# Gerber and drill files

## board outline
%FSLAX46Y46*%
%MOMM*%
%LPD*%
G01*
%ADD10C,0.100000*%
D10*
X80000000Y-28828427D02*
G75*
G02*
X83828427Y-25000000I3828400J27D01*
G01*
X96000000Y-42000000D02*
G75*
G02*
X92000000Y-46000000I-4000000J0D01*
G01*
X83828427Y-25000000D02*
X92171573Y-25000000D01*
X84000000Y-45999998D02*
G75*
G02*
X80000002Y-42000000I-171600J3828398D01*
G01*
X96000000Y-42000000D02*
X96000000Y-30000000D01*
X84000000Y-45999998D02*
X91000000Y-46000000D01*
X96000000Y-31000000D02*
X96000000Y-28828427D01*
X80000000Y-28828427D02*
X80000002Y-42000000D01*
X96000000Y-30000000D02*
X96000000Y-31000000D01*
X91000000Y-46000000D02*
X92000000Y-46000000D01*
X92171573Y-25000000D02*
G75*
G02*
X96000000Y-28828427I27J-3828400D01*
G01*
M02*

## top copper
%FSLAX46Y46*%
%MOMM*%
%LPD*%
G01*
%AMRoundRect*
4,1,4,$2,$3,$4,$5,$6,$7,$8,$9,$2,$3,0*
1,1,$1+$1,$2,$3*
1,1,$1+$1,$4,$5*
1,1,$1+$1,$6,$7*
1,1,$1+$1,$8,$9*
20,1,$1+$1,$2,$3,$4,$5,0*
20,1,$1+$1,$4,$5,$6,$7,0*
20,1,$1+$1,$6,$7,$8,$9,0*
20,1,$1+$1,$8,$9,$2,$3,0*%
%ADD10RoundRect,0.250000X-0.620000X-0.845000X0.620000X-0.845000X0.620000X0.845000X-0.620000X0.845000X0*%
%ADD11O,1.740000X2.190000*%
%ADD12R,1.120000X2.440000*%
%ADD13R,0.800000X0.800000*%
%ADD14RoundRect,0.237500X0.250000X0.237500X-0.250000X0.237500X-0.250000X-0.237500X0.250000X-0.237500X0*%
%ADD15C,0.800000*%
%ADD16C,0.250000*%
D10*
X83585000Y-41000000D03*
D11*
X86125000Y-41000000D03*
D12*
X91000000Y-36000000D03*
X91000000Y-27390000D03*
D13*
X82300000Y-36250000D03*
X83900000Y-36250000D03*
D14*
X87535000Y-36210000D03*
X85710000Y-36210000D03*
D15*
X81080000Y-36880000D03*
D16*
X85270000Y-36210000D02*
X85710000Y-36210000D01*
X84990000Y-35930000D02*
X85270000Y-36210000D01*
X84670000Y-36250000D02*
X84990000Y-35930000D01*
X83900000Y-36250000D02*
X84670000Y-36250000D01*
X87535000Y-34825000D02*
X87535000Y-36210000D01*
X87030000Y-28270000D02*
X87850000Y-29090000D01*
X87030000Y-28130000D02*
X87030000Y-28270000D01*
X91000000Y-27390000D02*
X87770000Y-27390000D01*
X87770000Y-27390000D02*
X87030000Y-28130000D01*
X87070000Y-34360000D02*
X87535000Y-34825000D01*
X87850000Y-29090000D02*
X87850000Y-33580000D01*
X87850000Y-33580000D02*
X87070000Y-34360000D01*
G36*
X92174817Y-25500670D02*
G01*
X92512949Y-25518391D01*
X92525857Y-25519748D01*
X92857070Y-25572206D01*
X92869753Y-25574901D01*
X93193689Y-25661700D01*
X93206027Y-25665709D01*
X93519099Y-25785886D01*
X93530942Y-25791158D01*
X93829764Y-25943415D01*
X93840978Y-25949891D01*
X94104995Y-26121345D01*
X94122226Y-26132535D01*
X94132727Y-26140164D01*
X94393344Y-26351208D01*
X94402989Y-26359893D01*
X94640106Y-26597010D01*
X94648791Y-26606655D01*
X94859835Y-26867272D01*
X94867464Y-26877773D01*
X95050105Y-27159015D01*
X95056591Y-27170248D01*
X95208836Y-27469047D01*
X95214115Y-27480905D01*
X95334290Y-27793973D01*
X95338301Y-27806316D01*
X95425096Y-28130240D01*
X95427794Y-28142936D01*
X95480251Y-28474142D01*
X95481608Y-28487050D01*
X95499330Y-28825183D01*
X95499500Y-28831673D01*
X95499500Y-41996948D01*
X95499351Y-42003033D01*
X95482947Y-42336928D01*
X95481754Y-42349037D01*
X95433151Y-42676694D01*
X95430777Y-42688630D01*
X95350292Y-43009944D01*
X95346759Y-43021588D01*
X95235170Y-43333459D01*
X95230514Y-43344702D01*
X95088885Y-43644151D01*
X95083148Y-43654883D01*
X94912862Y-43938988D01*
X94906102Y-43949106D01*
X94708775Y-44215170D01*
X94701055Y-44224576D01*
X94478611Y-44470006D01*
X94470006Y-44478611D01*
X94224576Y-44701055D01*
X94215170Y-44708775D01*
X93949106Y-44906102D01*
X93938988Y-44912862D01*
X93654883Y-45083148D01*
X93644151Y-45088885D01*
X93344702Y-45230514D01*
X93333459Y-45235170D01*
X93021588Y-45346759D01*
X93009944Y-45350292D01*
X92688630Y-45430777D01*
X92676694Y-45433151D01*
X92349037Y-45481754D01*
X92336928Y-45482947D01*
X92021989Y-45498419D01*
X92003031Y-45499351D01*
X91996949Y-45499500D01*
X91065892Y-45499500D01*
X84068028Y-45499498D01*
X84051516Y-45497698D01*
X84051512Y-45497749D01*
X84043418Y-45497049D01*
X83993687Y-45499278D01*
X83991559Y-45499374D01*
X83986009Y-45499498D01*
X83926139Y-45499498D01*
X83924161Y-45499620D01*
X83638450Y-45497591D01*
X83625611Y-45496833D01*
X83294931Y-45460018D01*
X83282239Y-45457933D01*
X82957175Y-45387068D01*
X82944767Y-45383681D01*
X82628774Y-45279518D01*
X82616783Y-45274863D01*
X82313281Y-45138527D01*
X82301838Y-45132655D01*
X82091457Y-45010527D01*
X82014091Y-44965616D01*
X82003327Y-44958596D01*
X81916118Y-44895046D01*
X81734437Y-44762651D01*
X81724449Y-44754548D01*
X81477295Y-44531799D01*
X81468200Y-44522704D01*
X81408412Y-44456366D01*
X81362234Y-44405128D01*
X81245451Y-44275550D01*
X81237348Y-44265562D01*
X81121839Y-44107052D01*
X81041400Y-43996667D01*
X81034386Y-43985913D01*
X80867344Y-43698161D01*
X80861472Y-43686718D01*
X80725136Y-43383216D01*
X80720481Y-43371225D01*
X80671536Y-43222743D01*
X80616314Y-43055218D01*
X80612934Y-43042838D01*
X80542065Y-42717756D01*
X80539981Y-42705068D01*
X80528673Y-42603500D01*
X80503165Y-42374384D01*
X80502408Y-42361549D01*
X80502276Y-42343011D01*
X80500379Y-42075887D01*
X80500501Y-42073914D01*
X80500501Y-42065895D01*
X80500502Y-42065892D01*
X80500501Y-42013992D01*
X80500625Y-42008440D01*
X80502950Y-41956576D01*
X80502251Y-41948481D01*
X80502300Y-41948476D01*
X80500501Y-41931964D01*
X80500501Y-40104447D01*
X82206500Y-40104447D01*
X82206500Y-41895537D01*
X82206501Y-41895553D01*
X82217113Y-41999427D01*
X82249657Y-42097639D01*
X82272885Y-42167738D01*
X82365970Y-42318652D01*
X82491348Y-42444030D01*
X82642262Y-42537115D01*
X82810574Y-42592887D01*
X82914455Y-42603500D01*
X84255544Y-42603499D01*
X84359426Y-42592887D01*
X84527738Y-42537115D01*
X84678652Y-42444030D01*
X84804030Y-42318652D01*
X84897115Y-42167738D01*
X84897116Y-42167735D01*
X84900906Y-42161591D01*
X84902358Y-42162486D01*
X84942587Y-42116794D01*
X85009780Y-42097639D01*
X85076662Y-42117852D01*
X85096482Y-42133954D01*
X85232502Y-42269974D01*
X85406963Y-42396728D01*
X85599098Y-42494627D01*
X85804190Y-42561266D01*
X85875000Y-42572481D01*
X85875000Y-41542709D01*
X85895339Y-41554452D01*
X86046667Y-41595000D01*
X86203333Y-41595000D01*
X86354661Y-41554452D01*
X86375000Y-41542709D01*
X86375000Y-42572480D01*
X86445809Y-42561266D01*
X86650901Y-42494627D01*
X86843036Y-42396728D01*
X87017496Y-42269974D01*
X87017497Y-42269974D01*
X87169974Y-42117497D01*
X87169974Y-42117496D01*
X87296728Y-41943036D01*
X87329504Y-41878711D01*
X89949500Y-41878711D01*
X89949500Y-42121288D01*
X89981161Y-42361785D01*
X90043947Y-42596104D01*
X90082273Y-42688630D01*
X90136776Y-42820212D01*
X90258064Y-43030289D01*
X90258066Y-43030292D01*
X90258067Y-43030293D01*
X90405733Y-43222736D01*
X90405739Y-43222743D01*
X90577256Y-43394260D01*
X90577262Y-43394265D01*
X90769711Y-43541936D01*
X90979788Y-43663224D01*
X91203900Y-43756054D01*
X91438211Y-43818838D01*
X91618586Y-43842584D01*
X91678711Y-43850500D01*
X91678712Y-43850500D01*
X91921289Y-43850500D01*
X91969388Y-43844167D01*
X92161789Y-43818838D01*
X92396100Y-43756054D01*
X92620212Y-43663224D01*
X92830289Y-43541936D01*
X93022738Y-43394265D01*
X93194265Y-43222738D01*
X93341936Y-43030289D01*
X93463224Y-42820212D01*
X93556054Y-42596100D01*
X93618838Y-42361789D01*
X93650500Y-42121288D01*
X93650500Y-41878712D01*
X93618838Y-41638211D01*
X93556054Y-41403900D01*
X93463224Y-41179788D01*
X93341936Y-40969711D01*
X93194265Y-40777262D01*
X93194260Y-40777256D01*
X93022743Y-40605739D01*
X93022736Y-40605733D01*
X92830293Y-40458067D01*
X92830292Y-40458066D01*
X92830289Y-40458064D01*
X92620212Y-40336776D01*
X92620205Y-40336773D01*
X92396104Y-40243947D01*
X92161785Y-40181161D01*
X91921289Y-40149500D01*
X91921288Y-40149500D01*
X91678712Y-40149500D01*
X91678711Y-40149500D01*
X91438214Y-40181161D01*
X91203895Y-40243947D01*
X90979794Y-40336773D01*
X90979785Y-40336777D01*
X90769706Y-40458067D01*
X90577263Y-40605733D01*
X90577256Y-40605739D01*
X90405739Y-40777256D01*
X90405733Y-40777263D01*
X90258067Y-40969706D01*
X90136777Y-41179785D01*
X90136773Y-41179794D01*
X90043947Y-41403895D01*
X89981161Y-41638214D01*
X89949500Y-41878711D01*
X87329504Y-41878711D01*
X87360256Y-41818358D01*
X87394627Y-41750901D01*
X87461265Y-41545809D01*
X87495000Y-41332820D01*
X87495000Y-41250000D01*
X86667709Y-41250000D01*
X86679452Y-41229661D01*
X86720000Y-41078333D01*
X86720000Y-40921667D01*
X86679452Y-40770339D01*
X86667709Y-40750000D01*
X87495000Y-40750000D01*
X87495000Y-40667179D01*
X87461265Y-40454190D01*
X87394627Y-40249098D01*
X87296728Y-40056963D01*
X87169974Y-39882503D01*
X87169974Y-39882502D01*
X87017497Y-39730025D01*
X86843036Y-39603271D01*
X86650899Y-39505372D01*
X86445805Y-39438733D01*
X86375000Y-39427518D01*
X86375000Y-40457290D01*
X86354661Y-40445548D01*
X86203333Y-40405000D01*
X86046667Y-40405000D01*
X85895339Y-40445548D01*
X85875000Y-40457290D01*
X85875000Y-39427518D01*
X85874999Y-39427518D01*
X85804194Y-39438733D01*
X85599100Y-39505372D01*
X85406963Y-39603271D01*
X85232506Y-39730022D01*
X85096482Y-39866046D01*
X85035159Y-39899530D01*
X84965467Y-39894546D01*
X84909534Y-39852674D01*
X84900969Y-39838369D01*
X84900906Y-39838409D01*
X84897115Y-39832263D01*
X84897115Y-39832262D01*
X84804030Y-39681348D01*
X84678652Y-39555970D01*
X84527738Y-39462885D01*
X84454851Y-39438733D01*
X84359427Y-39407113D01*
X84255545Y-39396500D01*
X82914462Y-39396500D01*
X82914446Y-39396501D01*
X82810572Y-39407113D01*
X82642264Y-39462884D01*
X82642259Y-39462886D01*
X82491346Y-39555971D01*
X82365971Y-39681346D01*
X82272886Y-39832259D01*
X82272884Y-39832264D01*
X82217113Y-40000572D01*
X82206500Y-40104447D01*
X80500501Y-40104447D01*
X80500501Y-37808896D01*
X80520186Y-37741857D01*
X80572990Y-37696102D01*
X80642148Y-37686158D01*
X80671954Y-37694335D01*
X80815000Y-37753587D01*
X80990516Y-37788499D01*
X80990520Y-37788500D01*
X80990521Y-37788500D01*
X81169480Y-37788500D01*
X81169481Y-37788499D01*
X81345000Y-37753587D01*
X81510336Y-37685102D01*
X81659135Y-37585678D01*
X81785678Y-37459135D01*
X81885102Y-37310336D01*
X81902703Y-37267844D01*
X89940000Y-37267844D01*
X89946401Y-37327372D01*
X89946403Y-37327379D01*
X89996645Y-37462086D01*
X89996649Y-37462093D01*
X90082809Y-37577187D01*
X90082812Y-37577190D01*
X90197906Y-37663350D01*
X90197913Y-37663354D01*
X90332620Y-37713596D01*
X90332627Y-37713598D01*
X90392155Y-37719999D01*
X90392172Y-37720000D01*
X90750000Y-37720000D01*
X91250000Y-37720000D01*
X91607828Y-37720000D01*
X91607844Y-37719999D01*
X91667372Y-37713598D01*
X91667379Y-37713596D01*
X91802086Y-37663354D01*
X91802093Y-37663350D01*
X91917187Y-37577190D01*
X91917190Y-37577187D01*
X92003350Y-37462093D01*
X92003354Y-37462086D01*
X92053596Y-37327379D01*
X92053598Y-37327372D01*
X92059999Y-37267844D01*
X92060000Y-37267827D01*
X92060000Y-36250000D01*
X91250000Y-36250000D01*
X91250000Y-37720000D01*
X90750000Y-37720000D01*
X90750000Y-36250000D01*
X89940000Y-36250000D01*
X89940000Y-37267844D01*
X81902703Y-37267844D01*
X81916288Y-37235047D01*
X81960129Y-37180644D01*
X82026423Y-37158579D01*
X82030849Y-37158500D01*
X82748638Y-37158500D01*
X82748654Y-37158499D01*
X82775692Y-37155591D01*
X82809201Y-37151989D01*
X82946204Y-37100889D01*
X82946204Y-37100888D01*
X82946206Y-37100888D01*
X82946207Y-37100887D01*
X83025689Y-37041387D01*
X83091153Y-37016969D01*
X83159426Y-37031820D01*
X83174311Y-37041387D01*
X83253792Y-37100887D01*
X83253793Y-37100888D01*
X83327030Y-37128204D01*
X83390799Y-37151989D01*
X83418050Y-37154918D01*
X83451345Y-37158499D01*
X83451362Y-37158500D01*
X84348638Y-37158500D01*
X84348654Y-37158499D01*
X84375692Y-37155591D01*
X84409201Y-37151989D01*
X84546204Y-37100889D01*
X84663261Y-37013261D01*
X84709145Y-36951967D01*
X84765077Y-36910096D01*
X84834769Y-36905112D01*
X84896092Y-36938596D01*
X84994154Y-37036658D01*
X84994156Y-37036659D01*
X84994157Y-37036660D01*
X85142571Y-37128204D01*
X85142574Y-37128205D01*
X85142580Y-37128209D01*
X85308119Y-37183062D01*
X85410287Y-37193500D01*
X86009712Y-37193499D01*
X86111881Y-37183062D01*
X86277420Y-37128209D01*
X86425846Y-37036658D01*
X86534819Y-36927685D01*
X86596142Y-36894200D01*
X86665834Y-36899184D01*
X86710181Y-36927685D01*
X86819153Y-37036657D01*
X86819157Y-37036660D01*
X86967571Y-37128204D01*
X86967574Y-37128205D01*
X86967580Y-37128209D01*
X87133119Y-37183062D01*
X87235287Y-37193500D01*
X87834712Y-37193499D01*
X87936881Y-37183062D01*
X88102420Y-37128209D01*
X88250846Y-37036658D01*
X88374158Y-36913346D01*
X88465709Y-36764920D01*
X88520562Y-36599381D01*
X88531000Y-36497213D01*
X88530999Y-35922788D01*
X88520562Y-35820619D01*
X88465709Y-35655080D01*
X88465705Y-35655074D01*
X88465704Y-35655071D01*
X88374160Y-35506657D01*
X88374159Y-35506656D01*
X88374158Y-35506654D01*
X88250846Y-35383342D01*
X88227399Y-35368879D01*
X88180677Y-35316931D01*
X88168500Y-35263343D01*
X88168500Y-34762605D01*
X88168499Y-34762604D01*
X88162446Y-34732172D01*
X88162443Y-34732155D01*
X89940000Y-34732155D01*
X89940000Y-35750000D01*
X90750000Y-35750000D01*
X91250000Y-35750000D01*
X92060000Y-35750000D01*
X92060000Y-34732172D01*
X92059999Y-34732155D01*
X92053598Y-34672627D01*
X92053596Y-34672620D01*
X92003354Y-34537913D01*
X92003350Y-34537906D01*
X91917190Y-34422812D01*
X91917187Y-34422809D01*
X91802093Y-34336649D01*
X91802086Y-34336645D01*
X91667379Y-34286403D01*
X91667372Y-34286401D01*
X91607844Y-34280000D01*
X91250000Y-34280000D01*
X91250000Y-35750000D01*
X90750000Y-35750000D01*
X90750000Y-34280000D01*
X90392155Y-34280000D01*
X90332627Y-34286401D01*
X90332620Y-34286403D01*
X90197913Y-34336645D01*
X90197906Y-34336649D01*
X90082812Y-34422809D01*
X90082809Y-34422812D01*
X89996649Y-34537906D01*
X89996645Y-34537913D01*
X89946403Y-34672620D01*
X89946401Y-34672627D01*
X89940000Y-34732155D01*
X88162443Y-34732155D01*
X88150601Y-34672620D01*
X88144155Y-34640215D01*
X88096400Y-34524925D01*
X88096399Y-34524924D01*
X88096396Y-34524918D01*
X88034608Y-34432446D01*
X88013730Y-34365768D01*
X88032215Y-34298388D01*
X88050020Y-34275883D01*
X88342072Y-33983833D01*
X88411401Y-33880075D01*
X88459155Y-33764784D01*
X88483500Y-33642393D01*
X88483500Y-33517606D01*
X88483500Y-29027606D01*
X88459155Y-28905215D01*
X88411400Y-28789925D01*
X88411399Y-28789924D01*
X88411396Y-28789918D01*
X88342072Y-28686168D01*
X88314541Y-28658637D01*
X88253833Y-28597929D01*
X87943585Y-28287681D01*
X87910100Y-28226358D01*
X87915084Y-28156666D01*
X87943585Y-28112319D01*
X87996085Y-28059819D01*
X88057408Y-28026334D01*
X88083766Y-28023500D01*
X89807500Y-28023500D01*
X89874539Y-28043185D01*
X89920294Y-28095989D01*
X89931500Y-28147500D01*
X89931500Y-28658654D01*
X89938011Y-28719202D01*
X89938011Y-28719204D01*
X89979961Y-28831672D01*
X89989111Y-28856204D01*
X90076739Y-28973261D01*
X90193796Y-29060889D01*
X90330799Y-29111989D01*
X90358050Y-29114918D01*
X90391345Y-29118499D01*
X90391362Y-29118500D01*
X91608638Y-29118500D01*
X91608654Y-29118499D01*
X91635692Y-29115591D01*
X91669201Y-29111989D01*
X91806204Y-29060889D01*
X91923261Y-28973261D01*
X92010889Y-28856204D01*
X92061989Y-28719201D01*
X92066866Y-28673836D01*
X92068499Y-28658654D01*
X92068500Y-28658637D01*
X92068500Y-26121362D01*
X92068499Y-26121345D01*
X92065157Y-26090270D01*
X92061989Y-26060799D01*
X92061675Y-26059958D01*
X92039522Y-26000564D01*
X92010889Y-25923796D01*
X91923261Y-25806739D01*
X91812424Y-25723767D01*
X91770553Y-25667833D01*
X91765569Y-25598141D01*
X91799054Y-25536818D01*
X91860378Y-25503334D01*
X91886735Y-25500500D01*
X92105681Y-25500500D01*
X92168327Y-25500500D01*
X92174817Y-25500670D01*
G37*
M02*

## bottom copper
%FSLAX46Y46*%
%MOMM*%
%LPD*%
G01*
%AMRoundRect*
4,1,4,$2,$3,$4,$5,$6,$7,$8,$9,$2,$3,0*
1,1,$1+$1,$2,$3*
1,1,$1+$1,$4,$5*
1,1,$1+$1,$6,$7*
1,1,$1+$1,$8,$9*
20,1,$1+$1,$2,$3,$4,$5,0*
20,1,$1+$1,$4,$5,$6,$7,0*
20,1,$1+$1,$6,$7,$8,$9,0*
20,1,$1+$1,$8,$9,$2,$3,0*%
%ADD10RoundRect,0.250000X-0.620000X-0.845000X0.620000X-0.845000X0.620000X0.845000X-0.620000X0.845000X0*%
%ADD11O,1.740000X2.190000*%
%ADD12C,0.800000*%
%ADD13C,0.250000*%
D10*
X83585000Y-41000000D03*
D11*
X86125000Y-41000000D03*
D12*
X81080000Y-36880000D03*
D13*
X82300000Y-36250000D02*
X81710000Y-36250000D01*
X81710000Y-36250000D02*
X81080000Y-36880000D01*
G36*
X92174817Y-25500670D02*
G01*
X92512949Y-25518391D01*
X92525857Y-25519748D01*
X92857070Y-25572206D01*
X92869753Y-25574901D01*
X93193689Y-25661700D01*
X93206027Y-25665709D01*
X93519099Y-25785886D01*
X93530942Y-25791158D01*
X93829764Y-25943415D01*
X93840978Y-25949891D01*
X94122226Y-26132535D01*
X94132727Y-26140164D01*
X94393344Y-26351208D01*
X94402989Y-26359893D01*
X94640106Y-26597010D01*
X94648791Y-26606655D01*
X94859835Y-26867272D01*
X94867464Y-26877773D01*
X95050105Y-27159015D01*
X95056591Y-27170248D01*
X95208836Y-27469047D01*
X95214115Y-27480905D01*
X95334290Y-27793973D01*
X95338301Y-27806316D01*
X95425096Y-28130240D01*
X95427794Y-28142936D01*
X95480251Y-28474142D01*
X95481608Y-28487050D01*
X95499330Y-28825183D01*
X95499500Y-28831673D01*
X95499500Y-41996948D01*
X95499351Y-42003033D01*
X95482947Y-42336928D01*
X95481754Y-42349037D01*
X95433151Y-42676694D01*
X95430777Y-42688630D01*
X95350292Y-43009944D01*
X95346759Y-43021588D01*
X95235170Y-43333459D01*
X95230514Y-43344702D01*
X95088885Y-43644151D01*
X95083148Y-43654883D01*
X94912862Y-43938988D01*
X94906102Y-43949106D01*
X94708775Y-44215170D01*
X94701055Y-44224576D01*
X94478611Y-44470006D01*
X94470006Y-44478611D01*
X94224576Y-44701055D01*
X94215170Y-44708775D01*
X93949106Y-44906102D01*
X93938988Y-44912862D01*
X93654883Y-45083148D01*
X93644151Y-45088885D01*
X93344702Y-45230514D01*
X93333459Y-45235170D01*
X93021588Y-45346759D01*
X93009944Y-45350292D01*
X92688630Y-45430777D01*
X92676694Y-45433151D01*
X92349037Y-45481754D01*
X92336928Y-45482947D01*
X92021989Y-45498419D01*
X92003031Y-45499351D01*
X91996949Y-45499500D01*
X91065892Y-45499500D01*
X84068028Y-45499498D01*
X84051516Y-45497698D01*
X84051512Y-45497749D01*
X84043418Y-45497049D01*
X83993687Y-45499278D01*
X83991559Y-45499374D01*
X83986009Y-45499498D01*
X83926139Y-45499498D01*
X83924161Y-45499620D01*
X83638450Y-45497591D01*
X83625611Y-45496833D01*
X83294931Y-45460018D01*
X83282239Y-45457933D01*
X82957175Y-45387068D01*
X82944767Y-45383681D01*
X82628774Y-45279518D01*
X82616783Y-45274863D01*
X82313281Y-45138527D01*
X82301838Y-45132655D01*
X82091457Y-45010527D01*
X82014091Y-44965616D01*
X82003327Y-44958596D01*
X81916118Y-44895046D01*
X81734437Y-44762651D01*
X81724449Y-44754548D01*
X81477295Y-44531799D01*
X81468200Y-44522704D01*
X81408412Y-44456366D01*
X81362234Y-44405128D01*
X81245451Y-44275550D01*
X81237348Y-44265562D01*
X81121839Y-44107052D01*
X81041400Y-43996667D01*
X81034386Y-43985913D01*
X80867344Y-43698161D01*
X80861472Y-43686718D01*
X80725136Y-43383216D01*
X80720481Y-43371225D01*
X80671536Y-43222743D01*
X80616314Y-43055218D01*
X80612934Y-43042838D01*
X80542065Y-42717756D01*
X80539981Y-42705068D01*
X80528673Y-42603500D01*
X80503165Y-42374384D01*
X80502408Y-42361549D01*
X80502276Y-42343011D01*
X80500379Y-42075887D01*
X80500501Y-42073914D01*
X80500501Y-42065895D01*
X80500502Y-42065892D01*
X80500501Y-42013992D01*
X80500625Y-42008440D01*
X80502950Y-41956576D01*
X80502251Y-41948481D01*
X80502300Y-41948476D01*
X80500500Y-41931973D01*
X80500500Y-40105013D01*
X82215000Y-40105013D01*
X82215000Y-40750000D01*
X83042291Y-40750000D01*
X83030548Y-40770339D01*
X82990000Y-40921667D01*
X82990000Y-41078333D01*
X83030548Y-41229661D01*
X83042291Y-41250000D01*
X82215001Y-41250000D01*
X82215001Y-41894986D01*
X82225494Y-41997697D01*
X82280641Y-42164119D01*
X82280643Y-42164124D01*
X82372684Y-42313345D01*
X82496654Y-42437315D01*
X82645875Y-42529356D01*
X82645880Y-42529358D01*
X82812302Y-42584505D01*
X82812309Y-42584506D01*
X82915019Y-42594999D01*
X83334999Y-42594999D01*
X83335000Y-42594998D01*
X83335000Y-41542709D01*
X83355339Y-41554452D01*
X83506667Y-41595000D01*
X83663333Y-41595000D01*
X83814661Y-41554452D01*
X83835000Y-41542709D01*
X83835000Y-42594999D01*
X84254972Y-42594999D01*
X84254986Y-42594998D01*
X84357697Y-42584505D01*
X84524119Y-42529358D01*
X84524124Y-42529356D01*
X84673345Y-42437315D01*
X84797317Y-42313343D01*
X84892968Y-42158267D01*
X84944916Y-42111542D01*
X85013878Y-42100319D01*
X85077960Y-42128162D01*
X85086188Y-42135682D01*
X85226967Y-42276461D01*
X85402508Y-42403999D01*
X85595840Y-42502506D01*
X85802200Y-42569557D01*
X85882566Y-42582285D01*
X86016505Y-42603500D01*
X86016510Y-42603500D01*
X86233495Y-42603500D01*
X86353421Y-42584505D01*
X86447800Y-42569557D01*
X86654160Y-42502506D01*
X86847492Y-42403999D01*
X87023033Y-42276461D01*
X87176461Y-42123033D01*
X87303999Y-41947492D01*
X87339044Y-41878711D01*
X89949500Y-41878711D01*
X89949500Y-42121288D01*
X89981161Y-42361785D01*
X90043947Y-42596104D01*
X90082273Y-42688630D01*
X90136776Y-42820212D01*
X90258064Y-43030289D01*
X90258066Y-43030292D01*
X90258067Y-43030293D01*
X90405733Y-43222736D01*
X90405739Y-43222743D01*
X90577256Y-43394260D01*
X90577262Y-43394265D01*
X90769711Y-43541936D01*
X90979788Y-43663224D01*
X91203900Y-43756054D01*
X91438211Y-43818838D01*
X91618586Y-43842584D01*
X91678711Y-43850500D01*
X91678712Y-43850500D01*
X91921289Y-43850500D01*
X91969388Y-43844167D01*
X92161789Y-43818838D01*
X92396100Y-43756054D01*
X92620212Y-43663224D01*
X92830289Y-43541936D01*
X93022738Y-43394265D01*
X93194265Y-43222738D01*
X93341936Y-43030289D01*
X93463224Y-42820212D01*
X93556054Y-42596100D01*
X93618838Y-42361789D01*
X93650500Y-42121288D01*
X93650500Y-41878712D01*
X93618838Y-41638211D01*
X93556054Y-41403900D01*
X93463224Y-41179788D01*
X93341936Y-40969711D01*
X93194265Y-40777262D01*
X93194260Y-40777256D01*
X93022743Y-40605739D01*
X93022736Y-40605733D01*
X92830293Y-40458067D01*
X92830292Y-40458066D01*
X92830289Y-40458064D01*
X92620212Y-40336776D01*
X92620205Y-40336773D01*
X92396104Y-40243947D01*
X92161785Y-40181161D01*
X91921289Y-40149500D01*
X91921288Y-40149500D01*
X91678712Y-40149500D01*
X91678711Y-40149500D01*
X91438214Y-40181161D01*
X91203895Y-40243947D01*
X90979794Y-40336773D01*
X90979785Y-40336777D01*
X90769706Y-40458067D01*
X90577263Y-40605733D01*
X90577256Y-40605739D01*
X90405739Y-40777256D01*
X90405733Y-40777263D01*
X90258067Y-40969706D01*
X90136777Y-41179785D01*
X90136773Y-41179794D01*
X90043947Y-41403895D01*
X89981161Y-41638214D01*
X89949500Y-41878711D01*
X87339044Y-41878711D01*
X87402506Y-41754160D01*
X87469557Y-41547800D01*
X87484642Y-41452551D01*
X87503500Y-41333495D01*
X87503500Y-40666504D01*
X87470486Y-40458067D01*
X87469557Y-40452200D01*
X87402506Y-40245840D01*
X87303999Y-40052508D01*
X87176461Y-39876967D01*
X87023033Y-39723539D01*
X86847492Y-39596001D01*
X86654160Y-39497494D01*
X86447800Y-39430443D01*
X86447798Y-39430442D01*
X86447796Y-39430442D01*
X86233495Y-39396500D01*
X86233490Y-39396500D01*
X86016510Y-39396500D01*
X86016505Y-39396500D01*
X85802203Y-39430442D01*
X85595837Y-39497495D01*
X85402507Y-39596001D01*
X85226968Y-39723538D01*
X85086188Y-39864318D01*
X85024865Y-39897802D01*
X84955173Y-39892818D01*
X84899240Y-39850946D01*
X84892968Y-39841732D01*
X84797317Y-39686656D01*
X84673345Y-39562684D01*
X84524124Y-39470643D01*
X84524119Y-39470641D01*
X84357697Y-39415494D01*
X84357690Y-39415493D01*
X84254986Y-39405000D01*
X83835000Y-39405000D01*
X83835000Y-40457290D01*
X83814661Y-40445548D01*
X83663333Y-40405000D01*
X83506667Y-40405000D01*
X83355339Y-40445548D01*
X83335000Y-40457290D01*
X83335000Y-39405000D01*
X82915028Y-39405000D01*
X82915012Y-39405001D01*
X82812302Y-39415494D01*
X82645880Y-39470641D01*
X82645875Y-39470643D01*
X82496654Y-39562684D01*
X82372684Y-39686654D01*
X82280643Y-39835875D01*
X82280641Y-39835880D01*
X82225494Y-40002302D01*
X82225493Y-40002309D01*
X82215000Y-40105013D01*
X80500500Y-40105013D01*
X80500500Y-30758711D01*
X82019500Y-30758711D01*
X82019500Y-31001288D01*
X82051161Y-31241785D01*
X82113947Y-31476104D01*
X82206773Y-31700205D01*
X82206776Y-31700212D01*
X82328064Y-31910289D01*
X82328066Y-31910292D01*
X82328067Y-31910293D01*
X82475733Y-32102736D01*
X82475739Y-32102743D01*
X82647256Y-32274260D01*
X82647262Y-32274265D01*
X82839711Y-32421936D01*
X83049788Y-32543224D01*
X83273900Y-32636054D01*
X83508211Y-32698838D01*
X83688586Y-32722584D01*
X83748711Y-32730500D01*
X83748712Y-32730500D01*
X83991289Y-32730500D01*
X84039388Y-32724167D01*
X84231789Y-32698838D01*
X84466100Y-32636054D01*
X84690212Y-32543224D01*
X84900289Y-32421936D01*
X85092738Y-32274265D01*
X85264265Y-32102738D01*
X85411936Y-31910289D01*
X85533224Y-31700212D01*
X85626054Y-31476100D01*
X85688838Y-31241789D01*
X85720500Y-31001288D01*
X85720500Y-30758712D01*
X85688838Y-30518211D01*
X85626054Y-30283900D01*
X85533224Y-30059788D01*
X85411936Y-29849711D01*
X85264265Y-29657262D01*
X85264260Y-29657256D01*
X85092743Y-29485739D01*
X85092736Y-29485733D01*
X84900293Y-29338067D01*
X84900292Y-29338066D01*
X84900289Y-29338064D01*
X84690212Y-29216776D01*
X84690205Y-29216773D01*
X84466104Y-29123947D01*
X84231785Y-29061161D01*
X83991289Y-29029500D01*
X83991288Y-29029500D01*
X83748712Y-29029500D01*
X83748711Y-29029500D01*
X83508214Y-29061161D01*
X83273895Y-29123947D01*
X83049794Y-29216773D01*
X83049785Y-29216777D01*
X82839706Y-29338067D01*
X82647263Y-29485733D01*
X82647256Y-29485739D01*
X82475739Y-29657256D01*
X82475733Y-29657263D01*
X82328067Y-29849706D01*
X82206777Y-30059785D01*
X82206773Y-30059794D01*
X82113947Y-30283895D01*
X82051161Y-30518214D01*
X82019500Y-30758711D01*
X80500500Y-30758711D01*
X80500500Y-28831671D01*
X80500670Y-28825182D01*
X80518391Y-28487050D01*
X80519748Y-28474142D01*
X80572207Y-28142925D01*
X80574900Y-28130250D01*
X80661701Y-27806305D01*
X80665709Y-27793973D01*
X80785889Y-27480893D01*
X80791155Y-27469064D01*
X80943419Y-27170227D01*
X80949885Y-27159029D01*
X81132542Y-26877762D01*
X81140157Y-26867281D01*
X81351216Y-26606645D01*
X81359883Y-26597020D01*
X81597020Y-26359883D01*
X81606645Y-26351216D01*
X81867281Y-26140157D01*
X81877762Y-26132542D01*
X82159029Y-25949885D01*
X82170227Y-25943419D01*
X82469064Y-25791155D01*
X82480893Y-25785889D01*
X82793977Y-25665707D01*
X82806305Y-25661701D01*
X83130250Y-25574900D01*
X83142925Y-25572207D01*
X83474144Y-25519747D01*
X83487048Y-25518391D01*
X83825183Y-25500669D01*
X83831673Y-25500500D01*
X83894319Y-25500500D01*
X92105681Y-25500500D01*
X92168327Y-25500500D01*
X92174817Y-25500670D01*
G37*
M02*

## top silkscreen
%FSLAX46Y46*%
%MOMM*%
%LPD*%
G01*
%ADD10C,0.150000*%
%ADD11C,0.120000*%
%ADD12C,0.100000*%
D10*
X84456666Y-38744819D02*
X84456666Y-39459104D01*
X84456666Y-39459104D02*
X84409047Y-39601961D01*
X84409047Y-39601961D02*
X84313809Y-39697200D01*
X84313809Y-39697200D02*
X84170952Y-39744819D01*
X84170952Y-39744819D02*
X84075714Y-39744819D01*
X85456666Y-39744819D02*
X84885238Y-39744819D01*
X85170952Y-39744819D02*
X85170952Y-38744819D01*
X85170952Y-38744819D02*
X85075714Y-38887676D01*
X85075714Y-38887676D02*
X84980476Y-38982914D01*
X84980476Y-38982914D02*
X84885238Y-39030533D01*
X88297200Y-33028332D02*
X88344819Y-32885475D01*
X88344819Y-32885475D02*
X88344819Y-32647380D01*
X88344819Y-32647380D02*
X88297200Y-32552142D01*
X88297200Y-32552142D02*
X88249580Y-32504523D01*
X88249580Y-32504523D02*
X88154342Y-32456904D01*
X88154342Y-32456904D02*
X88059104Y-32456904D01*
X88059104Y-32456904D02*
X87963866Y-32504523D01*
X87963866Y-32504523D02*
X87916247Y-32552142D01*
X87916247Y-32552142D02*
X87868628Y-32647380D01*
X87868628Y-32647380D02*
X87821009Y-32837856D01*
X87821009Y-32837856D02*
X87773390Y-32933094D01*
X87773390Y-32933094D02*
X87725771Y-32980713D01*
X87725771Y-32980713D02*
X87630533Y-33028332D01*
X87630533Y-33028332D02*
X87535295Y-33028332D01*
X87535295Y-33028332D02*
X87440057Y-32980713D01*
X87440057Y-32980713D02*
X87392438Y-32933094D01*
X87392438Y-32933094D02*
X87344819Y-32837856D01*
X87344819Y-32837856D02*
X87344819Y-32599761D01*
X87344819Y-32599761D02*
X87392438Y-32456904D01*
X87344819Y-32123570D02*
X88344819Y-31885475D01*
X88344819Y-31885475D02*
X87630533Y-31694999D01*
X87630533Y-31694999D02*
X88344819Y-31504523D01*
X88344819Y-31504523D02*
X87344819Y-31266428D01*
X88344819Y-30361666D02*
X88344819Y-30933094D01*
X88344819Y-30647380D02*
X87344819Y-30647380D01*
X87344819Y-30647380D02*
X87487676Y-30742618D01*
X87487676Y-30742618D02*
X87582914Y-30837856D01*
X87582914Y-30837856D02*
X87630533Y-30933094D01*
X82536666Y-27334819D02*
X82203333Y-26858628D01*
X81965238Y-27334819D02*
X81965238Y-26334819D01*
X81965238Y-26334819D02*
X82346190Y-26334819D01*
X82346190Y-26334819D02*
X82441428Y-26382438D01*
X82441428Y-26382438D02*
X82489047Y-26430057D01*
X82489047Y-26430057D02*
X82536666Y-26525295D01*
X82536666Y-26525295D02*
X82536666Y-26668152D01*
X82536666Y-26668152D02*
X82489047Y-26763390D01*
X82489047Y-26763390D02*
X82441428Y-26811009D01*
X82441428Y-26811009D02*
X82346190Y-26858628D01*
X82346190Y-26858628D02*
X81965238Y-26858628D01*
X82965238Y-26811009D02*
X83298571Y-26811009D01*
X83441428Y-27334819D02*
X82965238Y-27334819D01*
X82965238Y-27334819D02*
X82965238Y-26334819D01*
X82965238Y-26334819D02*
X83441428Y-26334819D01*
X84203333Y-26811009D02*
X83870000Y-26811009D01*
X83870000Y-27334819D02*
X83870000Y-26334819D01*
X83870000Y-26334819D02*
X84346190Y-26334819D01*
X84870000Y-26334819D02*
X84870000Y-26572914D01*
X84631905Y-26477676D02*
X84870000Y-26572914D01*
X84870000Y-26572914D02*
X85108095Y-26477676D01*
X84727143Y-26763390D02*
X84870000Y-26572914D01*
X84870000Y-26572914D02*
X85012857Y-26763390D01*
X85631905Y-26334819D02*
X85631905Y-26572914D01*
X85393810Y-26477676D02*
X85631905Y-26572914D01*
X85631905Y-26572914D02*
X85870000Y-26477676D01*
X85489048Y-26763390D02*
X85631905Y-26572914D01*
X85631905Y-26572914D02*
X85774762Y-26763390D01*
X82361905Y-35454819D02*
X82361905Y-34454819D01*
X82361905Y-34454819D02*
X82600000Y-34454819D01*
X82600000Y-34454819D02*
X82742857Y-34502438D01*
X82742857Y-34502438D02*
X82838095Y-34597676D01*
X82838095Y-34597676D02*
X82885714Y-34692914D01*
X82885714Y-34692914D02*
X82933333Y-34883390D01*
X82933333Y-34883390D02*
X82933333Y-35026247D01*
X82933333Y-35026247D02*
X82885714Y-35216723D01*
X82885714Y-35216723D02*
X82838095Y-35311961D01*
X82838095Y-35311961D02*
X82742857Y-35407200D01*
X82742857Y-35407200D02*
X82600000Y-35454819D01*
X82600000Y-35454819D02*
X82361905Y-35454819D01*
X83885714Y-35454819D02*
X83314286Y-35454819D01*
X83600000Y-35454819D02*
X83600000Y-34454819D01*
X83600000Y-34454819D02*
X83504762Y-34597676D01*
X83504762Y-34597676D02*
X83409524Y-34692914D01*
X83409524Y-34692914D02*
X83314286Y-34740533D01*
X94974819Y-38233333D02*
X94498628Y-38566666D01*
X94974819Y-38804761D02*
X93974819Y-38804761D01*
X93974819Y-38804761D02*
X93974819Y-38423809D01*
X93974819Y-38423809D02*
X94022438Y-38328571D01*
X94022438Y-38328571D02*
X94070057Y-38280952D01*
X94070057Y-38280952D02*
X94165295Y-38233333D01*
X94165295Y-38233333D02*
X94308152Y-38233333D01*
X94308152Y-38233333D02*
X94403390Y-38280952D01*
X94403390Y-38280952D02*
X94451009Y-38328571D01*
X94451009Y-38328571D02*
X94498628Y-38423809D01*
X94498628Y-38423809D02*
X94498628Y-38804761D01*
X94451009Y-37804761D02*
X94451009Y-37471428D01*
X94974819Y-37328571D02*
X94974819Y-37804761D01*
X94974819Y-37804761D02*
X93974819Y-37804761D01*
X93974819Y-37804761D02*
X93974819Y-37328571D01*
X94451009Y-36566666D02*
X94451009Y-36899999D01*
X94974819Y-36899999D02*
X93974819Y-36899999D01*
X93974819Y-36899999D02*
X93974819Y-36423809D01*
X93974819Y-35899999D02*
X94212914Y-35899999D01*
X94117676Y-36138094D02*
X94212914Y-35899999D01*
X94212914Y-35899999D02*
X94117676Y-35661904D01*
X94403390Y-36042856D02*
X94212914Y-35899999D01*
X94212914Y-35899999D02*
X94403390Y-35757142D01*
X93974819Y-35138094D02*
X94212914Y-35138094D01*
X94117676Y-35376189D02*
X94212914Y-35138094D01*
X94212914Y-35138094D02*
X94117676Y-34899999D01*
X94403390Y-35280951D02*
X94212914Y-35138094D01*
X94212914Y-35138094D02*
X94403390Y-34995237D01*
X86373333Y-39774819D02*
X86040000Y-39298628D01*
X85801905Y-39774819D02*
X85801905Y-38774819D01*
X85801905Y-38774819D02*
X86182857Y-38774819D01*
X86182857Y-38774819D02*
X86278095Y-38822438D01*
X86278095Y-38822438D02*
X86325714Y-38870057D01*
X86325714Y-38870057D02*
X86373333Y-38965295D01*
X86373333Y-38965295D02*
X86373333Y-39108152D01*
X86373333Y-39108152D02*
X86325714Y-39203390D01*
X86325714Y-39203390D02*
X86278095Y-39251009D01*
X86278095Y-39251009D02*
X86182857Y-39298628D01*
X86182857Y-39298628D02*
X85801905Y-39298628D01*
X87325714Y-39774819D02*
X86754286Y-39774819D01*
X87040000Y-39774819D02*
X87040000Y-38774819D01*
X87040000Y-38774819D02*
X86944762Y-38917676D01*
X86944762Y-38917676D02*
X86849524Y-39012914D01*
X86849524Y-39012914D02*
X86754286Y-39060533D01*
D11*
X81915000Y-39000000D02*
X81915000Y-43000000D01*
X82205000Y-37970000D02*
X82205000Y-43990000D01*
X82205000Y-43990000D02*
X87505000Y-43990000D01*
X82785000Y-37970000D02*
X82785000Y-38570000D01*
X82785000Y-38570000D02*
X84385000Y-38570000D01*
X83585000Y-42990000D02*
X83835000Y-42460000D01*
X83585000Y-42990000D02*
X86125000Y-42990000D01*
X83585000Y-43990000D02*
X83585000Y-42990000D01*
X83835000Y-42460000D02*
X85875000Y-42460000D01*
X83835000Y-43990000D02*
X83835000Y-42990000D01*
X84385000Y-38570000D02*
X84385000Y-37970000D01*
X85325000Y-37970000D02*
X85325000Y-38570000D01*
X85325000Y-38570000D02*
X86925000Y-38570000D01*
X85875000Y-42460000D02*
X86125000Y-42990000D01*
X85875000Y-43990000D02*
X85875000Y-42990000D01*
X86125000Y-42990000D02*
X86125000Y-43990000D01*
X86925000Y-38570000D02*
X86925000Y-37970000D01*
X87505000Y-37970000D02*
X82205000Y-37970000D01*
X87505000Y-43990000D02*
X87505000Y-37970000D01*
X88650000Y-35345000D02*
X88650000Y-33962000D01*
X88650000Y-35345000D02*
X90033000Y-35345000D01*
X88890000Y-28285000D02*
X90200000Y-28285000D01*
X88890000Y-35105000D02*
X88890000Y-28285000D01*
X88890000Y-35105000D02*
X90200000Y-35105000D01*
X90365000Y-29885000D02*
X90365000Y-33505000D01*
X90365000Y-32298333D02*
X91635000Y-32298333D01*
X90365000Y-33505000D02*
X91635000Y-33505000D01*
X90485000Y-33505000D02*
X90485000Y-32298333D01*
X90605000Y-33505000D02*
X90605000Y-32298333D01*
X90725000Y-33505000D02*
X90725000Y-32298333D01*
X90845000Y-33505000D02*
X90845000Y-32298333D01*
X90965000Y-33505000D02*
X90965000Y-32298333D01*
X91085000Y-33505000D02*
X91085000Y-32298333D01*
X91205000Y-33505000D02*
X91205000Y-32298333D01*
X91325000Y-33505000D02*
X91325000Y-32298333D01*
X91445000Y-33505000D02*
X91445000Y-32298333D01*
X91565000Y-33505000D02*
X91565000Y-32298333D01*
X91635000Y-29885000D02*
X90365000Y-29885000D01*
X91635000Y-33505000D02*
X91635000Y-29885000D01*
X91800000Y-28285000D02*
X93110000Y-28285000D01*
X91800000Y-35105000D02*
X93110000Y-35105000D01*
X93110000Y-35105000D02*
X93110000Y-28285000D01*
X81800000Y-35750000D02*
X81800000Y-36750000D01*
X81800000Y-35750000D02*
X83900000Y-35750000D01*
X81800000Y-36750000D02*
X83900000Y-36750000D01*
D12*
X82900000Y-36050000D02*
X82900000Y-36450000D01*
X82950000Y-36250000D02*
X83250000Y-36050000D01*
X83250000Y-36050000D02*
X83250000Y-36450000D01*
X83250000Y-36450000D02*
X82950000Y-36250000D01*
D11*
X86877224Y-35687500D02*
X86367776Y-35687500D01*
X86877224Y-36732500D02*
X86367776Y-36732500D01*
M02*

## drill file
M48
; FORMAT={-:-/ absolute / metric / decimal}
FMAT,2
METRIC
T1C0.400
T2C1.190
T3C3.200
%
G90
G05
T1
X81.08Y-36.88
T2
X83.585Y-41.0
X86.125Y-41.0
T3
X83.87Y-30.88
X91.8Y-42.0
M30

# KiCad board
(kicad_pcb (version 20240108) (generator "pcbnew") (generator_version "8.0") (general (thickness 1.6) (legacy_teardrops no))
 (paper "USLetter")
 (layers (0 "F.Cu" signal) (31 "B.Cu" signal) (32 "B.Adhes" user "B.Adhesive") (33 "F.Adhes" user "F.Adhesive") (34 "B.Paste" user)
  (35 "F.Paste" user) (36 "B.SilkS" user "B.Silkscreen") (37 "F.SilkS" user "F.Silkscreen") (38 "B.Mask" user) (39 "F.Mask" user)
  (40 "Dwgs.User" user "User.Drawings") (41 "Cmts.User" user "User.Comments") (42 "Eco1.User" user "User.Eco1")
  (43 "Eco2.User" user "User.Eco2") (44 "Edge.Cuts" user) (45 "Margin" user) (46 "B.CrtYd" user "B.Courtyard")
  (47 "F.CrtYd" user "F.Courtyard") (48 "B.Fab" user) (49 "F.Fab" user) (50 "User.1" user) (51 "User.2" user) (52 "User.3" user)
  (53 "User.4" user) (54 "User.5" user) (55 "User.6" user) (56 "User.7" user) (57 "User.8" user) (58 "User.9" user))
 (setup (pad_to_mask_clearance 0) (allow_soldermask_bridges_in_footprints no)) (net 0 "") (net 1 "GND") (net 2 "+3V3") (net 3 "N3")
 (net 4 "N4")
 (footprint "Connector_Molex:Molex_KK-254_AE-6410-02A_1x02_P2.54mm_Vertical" (layer "F.Cu") (at 83.585 41)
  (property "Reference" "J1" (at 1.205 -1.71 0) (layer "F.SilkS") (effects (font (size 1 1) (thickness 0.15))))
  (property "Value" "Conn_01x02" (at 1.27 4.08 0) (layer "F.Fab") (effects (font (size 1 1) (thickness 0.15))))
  (fp_line (start -1.67 -2) (end -1.67 2) (stroke (width 0.12) (type solid)) (layer "F.SilkS"))
  (fp_line (start -1.38 -3.03) (end -1.38 2.99) (stroke (width 0.12) (type solid)) (layer "F.SilkS"))
  (fp_line (start -1.38 2.99) (end 3.92 2.99) (stroke (width 0.12) (type solid)) (layer "F.SilkS"))
  (fp_line (start -0.8 -3.03) (end -0.8 -2.43) (stroke (width 0.12) (type solid)) (layer "F.SilkS"))
  (fp_line (start -0.8 -2.43) (end 0.8 -2.43) (stroke (width 0.12) (type solid)) (layer "F.SilkS"))
  (fp_line (start 0 1.99) (end 0.25 1.46) (stroke (width 0.12) (type solid)) (layer "F.SilkS"))
  (fp_line (start 0 1.99) (end 2.54 1.99) (stroke (width 0.12) (type solid)) (layer "F.SilkS"))
  (fp_line (start 0 2.99) (end 0 1.99) (stroke (width 0.12) (type solid)) (layer "F.SilkS"))
  (fp_line (start 0.25 1.46) (end 2.29 1.46) (stroke (width 0.12) (type solid)) (layer "F.SilkS"))
  (fp_line (start 0.25 2.99) (end 0.25 1.99) (stroke (width 0.12) (type solid)) (layer "F.SilkS"))
  (fp_line (start 0.8 -2.43) (end 0.8 -3.03) (stroke (width 0.12) (type solid)) (layer "F.SilkS"))
  (fp_line (start 1.74 -3.03) (end 1.74 -2.43) (stroke (width 0.12) (type solid)) (layer "F.SilkS"))
  (fp_line (start 1.74 -2.43) (end 3.34 -2.43) (stroke (width 0.12) (type solid)) (layer "F.SilkS"))
  (fp_line (start 2.29 1.46) (end 2.54 1.99) (stroke (width 0.12) (type solid)) (layer "F.SilkS"))
  (fp_line (start 2.29 2.99) (end 2.29 1.99) (stroke (width 0.12) (type solid)) (layer "F.SilkS"))
  (fp_line (start 2.54 1.99) (end 2.54 2.99) (stroke (width 0.12) (type solid)) (layer "F.SilkS"))
  (fp_line (start 3.34 -2.43) (end 3.34 -3.03) (stroke (width 0.12) (type solid)) (layer "F.SilkS"))
  (fp_line (start 3.92 -3.03) (end -1.38 -3.03) (stroke (width 0.12) (type solid)) (layer "F.SilkS"))
  (fp_line (start 3.92 2.99) (end 3.92 -3.03) (stroke (width 0.12) (type solid)) (layer "F.SilkS"))
  (pad "1" thru_hole roundrect (at 0 0) (size 1.74 2.19) (drill 1.19) (layers "*.Cu" "*.Mask") (remove_unused_layers no)
   (roundrect_rratio 0.143678) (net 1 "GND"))
  (pad "2" thru_hole oval (at 2.54 0) (size 1.74 2.19) (drill 1.19) (layers "*.Cu" "*.Mask") (remove_unused_layers no) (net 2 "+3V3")))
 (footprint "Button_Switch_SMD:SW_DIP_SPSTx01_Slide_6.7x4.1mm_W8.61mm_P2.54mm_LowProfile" (layer "F.Cu") (at 91 31.695 90)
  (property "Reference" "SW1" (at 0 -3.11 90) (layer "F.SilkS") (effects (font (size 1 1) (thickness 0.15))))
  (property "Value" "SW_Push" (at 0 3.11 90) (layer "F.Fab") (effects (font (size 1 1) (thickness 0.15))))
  (fp_line (start -3.65 -2.35) (end -2.267 -2.35) (stroke (width 0.12) (type solid)) (layer "F.SilkS"))
  (fp_line (start -3.65 -2.35) (end -3.65 -0.967) (stroke (width 0.12) (type solid)) (layer "F.SilkS"))
  (fp_line (start 3.41 -2.11) (end 3.41 -0.8) (stroke (width 0.12) (type solid)) (layer "F.SilkS"))
  (fp_line (start -3.41 -2.11) (end 3.41 -2.11) (stroke (width 0.12) (type solid)) (layer "F.SilkS"))
  (fp_line (start -3.41 -2.11) (end -3.41 -0.8) (stroke (width 0.12) (type solid)) (layer "F.SilkS"))
  (fp_line (start 1.81 -0.635) (end -1.81 -0.635) (stroke (width 0.12) (type solid)) (layer "F.SilkS"))
  (fp_line (start -0.603333 -0.635) (end -0.603333 0.635) (stroke (width 0.12) (type solid)) (layer "F.SilkS"))
  (fp_line (start -1.81 -0.635) (end -1.81 0.635) (stroke (width 0.12) (type solid)) (layer "F.SilkS"))
  (fp_line (start -1.81 -0.515) (end -0.603333 -0.515) (stroke (width 0.12) (type solid)) (layer "F.SilkS"))
  (fp_line (start -1.81 -0.395) (end -0.603333 -0.395) (stroke (width 0.12) (type solid)) (layer "F.SilkS"))
  (fp_line (start -1.81 -0.275) (end -0.603333 -0.275) (stroke (width 0.12) (type solid)) (layer "F.SilkS"))
  (fp_line (start -1.81 -0.155) (end -0.603333 -0.155) (stroke (width 0.12) (type solid)) (layer "F.SilkS"))
  (fp_line (start -1.81 -0.035) (end -0.603333 -0.035) (stroke (width 0.12) (type solid)) (layer "F.SilkS"))
  (fp_line (start -1.81 0.085) (end -0.603333 0.085) (stroke (width 0.12) (type solid)) (layer "F.SilkS"))
  (fp_line (start -1.81 0.205) (end -0.603333 0.205) (stroke (width 0.12) (type solid)) (layer "F.SilkS"))
  (fp_line (start -1.81 0.325) (end -0.603333 0.325) (stroke (width 0.12) (type solid)) (layer "F.SilkS"))
  (fp_line (start -1.81 0.445) (end -0.603333 0.445) (stroke (width 0.12) (type solid)) (layer "F.SilkS"))
  (fp_line (start -1.81 0.565) (end -0.603333 0.565) (stroke (width 0.12) (type solid)) (layer "F.SilkS"))
  (fp_line (start 1.81 0.635) (end 1.81 -0.635) (stroke (width 0.12) (type solid)) (layer "F.SilkS"))
  (fp_line (start -1.81 0.635) (end 1.81 0.635) (stroke (width 0.12) (type solid)) (layer "F.SilkS"))
  (fp_line (start 3.41 0.8) (end 3.41 2.11) (stroke (width 0.12) (type solid)) (layer "F.SilkS"))
  (fp_line (start -3.41 0.8) (end -3.41 2.11) (stroke (width 0.12) (type solid)) (layer "F.SilkS"))
  (fp_line (start -3.41 2.11) (end 3.41 2.11) (stroke (width 0.12) (type solid)) (layer "F.SilkS"))
  (pad "1" smd rect (at -4.305 0 90) (size 2.44 1.12) (layers "F.Cu" "F.Paste" "F.Mask") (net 2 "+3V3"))
  (pad "2" smd rect (at 4.305 0 90) (size 2.44 1.12) (layers "F.Cu" "F.Paste" "F.Mask") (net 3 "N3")))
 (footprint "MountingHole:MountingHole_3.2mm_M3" (layer "F.Cu") (at 83.87 30.88)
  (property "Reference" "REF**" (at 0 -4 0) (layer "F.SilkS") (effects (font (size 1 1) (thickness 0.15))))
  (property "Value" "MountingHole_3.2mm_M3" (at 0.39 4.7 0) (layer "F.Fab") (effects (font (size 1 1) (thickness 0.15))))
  (pad "" np_thru_hole circle (at 0 0) (size 3.2 3.2) (drill 3.2) (layers "F&B.Cu" "*.Mask")))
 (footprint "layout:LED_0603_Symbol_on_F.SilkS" (layer "F.Cu") (at 83.1 36.25)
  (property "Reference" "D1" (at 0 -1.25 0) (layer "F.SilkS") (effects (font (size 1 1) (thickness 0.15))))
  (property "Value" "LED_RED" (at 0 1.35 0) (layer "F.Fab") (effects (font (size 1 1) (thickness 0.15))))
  (fp_line (start -1.3 -0.5) (end -1.3 0.5) (stroke (width 0.12) (type solid)) (layer "F.SilkS"))
  (fp_line (start -1.3 -0.5) (end 0.8 -0.5) (stroke (width 0.12) (type solid)) (layer "F.SilkS"))
  (fp_line (start -1.3 0.5) (end 0.8 0.5) (stroke (width 0.12) (type solid)) (layer "F.SilkS"))
  (fp_line (start -0.2 -0.2) (end -0.2 0.2) (stroke (width 0.1) (type solid)) (layer "F.SilkS"))
  (fp_line (start -0.15 0) (end 0.15 -0.2) (stroke (width 0.1) (type solid)) (layer "F.SilkS"))
  (fp_line (start 0.15 -0.2) (end 0.15 0.2) (stroke (width 0.1) (type solid)) (layer "F.SilkS"))
  (fp_line (start 0.15 0.2) (end -0.15 0) (stroke (width 0.1) (type solid)) (layer "F.SilkS"))
  (pad "1" smd rect (at -0.8 0 180) (size 0.8 0.8) (layers "F.Cu" "F.Paste" "F.Mask") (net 1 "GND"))
  (pad "2" smd rect (at 0.8 0 180) (size 0.8 0.8) (layers "F.Cu" "F.Paste" "F.Mask") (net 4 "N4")))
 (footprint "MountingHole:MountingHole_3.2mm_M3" (layer "F.Cu") (at 91.8 42)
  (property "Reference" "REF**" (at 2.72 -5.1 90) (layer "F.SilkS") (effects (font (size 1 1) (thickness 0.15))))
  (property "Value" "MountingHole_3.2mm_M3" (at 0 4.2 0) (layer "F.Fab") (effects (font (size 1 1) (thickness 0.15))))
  (pad "" np_thru_hole circle (at 0 0) (size 3.2 3.2) (drill 3.2) (layers "F&B.Cu" "*.Mask")))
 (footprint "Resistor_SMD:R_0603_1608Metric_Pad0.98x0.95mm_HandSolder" (layer "F.Cu") (at 86.6225 36.21 180)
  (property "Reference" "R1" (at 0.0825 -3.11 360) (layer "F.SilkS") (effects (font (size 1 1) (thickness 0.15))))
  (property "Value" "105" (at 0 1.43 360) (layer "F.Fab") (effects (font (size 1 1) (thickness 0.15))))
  (fp_line (start -0.254724 0.5225) (end 0.254724 0.5225) (stroke (width 0.12) (type solid)) (layer "F.SilkS"))
  (fp_line (start -0.254724 -0.5225) (end 0.254724 -0.5225) (stroke (width 0.12) (type solid)) (layer "F.SilkS"))
  (pad "1" smd roundrect (at -0.9125 0 180) (size 0.975 0.95) (layers "F.Cu" "F.Paste" "F.Mask") (roundrect_rratio 0.25) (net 3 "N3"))
  (pad "2" smd roundrect (at 0.9125 0 180) (size 0.975 0.95) (layers "F.Cu" "F.Paste" "F.Mask") (roundrect_rratio 0.25) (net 4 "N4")))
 (gr_arc (start 80 28.828427) (mid 81.12132 26.12132) (end 83.828427 25) (stroke (width 0.1) (type default)) (layer "Edge.Cuts"))
 (gr_arc (start 96 42) (mid 94.828427 44.828427) (end 92 46) (stroke (width 0.1) (type default)) (layer "Edge.Cuts"))
 (gr_line (start 83.828427 25) (end 92.171573 25) (stroke (width 0.1) (type default)) (layer "Edge.Cuts"))
 (gr_arc (start 84 45.999998) (mid 81.118605 44.881395) (end 80.000002 42) (stroke (width 0.1) (type default)) (layer "Edge.Cuts"))
 (gr_line (start 96 42) (end 96 30) (stroke (width 0.1) (type default)) (layer "Edge.Cuts"))
 (gr_line (start 84 45.999998) (end 91 46) (stroke (width 0.1) (type default)) (layer "Edge.Cuts"))
 (gr_line (start 96 31) (end 96 28.828427) (stroke (width 0.1) (type default)) (layer "Edge.Cuts"))
 (gr_line (start 80 28.828427) (end 80.000002 42) (stroke (width 0.1) (type default)) (layer "Edge.Cuts"))
 (gr_line (start 96 30) (end 96 31) (stroke (width 0.1) (type default)) (layer "Edge.Cuts"))
 (gr_line (start 91 46) (end 92 46) (stroke (width 0.1) (type default)) (layer "Edge.Cuts"))
 (gr_arc (start 92.171573 25) (mid 94.87868 26.12132) (end 96 28.828427) (stroke (width 0.1) (type default)) (layer "Edge.Cuts"))
 (segment (start 85.27 36.21) (end 85.71 36.21) (width 0.25) (layer "F.Cu") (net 4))
 (segment (start 84.99 35.93) (end 85.27 36.21) (width 0.25) (layer "F.Cu") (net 4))
 (segment (start 84.67 36.25) (end 84.99 35.93) (width 0.25) (layer "F.Cu") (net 4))
 (segment (start 83.9 36.25) (end 84.67 36.25) (width 0.25) (layer "F.Cu") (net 4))
 (via (at 81.08 36.88) (size 0.8) (drill 0.4) (layers "F.Cu" "B.Cu") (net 1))
 (segment (start 82.3 36.25) (end 81.71 36.25) (width 0.25) (layer "B.Cu") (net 1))
 (segment (start 81.71 36.25) (end 81.08 36.88) (width 0.25) (layer "B.Cu") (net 1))
 (segment (start 87.535 34.825) (end 87.535 36.21) (width 0.25) (layer "F.Cu") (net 3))
 (segment (start 87.03 28.27) (end 87.85 29.09) (width 0.25) (layer "F.Cu") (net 3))
 (segment (start 87.03 28.13) (end 87.03 28.27) (width 0.25) (layer "F.Cu") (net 3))
 (segment (start 91 27.39) (end 87.77 27.39) (width 0.25) (layer "F.Cu") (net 3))
 (segment (start 87.77 27.39) (end 87.03 28.13) (width 0.25) (layer "F.Cu") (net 3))
 (segment (start 87.07 34.36) (end 87.535 34.825) (width 0.25) (layer "F.Cu") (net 3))
 (segment (start 87.85 29.09) (end 87.85 33.58) (width 0.25) (layer "F.Cu") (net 3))
 (segment (start 87.85 33.58) (end 87.07 34.36) (width 0.25) (layer "F.Cu") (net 3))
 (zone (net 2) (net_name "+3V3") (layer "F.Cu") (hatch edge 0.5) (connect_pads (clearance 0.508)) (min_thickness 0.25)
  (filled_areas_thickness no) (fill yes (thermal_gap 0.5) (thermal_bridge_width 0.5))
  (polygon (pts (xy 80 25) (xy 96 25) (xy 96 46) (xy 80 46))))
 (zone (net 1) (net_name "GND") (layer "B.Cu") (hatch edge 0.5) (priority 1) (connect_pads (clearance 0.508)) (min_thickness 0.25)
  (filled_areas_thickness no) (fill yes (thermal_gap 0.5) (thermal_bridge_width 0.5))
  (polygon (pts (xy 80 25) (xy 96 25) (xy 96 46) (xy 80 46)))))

